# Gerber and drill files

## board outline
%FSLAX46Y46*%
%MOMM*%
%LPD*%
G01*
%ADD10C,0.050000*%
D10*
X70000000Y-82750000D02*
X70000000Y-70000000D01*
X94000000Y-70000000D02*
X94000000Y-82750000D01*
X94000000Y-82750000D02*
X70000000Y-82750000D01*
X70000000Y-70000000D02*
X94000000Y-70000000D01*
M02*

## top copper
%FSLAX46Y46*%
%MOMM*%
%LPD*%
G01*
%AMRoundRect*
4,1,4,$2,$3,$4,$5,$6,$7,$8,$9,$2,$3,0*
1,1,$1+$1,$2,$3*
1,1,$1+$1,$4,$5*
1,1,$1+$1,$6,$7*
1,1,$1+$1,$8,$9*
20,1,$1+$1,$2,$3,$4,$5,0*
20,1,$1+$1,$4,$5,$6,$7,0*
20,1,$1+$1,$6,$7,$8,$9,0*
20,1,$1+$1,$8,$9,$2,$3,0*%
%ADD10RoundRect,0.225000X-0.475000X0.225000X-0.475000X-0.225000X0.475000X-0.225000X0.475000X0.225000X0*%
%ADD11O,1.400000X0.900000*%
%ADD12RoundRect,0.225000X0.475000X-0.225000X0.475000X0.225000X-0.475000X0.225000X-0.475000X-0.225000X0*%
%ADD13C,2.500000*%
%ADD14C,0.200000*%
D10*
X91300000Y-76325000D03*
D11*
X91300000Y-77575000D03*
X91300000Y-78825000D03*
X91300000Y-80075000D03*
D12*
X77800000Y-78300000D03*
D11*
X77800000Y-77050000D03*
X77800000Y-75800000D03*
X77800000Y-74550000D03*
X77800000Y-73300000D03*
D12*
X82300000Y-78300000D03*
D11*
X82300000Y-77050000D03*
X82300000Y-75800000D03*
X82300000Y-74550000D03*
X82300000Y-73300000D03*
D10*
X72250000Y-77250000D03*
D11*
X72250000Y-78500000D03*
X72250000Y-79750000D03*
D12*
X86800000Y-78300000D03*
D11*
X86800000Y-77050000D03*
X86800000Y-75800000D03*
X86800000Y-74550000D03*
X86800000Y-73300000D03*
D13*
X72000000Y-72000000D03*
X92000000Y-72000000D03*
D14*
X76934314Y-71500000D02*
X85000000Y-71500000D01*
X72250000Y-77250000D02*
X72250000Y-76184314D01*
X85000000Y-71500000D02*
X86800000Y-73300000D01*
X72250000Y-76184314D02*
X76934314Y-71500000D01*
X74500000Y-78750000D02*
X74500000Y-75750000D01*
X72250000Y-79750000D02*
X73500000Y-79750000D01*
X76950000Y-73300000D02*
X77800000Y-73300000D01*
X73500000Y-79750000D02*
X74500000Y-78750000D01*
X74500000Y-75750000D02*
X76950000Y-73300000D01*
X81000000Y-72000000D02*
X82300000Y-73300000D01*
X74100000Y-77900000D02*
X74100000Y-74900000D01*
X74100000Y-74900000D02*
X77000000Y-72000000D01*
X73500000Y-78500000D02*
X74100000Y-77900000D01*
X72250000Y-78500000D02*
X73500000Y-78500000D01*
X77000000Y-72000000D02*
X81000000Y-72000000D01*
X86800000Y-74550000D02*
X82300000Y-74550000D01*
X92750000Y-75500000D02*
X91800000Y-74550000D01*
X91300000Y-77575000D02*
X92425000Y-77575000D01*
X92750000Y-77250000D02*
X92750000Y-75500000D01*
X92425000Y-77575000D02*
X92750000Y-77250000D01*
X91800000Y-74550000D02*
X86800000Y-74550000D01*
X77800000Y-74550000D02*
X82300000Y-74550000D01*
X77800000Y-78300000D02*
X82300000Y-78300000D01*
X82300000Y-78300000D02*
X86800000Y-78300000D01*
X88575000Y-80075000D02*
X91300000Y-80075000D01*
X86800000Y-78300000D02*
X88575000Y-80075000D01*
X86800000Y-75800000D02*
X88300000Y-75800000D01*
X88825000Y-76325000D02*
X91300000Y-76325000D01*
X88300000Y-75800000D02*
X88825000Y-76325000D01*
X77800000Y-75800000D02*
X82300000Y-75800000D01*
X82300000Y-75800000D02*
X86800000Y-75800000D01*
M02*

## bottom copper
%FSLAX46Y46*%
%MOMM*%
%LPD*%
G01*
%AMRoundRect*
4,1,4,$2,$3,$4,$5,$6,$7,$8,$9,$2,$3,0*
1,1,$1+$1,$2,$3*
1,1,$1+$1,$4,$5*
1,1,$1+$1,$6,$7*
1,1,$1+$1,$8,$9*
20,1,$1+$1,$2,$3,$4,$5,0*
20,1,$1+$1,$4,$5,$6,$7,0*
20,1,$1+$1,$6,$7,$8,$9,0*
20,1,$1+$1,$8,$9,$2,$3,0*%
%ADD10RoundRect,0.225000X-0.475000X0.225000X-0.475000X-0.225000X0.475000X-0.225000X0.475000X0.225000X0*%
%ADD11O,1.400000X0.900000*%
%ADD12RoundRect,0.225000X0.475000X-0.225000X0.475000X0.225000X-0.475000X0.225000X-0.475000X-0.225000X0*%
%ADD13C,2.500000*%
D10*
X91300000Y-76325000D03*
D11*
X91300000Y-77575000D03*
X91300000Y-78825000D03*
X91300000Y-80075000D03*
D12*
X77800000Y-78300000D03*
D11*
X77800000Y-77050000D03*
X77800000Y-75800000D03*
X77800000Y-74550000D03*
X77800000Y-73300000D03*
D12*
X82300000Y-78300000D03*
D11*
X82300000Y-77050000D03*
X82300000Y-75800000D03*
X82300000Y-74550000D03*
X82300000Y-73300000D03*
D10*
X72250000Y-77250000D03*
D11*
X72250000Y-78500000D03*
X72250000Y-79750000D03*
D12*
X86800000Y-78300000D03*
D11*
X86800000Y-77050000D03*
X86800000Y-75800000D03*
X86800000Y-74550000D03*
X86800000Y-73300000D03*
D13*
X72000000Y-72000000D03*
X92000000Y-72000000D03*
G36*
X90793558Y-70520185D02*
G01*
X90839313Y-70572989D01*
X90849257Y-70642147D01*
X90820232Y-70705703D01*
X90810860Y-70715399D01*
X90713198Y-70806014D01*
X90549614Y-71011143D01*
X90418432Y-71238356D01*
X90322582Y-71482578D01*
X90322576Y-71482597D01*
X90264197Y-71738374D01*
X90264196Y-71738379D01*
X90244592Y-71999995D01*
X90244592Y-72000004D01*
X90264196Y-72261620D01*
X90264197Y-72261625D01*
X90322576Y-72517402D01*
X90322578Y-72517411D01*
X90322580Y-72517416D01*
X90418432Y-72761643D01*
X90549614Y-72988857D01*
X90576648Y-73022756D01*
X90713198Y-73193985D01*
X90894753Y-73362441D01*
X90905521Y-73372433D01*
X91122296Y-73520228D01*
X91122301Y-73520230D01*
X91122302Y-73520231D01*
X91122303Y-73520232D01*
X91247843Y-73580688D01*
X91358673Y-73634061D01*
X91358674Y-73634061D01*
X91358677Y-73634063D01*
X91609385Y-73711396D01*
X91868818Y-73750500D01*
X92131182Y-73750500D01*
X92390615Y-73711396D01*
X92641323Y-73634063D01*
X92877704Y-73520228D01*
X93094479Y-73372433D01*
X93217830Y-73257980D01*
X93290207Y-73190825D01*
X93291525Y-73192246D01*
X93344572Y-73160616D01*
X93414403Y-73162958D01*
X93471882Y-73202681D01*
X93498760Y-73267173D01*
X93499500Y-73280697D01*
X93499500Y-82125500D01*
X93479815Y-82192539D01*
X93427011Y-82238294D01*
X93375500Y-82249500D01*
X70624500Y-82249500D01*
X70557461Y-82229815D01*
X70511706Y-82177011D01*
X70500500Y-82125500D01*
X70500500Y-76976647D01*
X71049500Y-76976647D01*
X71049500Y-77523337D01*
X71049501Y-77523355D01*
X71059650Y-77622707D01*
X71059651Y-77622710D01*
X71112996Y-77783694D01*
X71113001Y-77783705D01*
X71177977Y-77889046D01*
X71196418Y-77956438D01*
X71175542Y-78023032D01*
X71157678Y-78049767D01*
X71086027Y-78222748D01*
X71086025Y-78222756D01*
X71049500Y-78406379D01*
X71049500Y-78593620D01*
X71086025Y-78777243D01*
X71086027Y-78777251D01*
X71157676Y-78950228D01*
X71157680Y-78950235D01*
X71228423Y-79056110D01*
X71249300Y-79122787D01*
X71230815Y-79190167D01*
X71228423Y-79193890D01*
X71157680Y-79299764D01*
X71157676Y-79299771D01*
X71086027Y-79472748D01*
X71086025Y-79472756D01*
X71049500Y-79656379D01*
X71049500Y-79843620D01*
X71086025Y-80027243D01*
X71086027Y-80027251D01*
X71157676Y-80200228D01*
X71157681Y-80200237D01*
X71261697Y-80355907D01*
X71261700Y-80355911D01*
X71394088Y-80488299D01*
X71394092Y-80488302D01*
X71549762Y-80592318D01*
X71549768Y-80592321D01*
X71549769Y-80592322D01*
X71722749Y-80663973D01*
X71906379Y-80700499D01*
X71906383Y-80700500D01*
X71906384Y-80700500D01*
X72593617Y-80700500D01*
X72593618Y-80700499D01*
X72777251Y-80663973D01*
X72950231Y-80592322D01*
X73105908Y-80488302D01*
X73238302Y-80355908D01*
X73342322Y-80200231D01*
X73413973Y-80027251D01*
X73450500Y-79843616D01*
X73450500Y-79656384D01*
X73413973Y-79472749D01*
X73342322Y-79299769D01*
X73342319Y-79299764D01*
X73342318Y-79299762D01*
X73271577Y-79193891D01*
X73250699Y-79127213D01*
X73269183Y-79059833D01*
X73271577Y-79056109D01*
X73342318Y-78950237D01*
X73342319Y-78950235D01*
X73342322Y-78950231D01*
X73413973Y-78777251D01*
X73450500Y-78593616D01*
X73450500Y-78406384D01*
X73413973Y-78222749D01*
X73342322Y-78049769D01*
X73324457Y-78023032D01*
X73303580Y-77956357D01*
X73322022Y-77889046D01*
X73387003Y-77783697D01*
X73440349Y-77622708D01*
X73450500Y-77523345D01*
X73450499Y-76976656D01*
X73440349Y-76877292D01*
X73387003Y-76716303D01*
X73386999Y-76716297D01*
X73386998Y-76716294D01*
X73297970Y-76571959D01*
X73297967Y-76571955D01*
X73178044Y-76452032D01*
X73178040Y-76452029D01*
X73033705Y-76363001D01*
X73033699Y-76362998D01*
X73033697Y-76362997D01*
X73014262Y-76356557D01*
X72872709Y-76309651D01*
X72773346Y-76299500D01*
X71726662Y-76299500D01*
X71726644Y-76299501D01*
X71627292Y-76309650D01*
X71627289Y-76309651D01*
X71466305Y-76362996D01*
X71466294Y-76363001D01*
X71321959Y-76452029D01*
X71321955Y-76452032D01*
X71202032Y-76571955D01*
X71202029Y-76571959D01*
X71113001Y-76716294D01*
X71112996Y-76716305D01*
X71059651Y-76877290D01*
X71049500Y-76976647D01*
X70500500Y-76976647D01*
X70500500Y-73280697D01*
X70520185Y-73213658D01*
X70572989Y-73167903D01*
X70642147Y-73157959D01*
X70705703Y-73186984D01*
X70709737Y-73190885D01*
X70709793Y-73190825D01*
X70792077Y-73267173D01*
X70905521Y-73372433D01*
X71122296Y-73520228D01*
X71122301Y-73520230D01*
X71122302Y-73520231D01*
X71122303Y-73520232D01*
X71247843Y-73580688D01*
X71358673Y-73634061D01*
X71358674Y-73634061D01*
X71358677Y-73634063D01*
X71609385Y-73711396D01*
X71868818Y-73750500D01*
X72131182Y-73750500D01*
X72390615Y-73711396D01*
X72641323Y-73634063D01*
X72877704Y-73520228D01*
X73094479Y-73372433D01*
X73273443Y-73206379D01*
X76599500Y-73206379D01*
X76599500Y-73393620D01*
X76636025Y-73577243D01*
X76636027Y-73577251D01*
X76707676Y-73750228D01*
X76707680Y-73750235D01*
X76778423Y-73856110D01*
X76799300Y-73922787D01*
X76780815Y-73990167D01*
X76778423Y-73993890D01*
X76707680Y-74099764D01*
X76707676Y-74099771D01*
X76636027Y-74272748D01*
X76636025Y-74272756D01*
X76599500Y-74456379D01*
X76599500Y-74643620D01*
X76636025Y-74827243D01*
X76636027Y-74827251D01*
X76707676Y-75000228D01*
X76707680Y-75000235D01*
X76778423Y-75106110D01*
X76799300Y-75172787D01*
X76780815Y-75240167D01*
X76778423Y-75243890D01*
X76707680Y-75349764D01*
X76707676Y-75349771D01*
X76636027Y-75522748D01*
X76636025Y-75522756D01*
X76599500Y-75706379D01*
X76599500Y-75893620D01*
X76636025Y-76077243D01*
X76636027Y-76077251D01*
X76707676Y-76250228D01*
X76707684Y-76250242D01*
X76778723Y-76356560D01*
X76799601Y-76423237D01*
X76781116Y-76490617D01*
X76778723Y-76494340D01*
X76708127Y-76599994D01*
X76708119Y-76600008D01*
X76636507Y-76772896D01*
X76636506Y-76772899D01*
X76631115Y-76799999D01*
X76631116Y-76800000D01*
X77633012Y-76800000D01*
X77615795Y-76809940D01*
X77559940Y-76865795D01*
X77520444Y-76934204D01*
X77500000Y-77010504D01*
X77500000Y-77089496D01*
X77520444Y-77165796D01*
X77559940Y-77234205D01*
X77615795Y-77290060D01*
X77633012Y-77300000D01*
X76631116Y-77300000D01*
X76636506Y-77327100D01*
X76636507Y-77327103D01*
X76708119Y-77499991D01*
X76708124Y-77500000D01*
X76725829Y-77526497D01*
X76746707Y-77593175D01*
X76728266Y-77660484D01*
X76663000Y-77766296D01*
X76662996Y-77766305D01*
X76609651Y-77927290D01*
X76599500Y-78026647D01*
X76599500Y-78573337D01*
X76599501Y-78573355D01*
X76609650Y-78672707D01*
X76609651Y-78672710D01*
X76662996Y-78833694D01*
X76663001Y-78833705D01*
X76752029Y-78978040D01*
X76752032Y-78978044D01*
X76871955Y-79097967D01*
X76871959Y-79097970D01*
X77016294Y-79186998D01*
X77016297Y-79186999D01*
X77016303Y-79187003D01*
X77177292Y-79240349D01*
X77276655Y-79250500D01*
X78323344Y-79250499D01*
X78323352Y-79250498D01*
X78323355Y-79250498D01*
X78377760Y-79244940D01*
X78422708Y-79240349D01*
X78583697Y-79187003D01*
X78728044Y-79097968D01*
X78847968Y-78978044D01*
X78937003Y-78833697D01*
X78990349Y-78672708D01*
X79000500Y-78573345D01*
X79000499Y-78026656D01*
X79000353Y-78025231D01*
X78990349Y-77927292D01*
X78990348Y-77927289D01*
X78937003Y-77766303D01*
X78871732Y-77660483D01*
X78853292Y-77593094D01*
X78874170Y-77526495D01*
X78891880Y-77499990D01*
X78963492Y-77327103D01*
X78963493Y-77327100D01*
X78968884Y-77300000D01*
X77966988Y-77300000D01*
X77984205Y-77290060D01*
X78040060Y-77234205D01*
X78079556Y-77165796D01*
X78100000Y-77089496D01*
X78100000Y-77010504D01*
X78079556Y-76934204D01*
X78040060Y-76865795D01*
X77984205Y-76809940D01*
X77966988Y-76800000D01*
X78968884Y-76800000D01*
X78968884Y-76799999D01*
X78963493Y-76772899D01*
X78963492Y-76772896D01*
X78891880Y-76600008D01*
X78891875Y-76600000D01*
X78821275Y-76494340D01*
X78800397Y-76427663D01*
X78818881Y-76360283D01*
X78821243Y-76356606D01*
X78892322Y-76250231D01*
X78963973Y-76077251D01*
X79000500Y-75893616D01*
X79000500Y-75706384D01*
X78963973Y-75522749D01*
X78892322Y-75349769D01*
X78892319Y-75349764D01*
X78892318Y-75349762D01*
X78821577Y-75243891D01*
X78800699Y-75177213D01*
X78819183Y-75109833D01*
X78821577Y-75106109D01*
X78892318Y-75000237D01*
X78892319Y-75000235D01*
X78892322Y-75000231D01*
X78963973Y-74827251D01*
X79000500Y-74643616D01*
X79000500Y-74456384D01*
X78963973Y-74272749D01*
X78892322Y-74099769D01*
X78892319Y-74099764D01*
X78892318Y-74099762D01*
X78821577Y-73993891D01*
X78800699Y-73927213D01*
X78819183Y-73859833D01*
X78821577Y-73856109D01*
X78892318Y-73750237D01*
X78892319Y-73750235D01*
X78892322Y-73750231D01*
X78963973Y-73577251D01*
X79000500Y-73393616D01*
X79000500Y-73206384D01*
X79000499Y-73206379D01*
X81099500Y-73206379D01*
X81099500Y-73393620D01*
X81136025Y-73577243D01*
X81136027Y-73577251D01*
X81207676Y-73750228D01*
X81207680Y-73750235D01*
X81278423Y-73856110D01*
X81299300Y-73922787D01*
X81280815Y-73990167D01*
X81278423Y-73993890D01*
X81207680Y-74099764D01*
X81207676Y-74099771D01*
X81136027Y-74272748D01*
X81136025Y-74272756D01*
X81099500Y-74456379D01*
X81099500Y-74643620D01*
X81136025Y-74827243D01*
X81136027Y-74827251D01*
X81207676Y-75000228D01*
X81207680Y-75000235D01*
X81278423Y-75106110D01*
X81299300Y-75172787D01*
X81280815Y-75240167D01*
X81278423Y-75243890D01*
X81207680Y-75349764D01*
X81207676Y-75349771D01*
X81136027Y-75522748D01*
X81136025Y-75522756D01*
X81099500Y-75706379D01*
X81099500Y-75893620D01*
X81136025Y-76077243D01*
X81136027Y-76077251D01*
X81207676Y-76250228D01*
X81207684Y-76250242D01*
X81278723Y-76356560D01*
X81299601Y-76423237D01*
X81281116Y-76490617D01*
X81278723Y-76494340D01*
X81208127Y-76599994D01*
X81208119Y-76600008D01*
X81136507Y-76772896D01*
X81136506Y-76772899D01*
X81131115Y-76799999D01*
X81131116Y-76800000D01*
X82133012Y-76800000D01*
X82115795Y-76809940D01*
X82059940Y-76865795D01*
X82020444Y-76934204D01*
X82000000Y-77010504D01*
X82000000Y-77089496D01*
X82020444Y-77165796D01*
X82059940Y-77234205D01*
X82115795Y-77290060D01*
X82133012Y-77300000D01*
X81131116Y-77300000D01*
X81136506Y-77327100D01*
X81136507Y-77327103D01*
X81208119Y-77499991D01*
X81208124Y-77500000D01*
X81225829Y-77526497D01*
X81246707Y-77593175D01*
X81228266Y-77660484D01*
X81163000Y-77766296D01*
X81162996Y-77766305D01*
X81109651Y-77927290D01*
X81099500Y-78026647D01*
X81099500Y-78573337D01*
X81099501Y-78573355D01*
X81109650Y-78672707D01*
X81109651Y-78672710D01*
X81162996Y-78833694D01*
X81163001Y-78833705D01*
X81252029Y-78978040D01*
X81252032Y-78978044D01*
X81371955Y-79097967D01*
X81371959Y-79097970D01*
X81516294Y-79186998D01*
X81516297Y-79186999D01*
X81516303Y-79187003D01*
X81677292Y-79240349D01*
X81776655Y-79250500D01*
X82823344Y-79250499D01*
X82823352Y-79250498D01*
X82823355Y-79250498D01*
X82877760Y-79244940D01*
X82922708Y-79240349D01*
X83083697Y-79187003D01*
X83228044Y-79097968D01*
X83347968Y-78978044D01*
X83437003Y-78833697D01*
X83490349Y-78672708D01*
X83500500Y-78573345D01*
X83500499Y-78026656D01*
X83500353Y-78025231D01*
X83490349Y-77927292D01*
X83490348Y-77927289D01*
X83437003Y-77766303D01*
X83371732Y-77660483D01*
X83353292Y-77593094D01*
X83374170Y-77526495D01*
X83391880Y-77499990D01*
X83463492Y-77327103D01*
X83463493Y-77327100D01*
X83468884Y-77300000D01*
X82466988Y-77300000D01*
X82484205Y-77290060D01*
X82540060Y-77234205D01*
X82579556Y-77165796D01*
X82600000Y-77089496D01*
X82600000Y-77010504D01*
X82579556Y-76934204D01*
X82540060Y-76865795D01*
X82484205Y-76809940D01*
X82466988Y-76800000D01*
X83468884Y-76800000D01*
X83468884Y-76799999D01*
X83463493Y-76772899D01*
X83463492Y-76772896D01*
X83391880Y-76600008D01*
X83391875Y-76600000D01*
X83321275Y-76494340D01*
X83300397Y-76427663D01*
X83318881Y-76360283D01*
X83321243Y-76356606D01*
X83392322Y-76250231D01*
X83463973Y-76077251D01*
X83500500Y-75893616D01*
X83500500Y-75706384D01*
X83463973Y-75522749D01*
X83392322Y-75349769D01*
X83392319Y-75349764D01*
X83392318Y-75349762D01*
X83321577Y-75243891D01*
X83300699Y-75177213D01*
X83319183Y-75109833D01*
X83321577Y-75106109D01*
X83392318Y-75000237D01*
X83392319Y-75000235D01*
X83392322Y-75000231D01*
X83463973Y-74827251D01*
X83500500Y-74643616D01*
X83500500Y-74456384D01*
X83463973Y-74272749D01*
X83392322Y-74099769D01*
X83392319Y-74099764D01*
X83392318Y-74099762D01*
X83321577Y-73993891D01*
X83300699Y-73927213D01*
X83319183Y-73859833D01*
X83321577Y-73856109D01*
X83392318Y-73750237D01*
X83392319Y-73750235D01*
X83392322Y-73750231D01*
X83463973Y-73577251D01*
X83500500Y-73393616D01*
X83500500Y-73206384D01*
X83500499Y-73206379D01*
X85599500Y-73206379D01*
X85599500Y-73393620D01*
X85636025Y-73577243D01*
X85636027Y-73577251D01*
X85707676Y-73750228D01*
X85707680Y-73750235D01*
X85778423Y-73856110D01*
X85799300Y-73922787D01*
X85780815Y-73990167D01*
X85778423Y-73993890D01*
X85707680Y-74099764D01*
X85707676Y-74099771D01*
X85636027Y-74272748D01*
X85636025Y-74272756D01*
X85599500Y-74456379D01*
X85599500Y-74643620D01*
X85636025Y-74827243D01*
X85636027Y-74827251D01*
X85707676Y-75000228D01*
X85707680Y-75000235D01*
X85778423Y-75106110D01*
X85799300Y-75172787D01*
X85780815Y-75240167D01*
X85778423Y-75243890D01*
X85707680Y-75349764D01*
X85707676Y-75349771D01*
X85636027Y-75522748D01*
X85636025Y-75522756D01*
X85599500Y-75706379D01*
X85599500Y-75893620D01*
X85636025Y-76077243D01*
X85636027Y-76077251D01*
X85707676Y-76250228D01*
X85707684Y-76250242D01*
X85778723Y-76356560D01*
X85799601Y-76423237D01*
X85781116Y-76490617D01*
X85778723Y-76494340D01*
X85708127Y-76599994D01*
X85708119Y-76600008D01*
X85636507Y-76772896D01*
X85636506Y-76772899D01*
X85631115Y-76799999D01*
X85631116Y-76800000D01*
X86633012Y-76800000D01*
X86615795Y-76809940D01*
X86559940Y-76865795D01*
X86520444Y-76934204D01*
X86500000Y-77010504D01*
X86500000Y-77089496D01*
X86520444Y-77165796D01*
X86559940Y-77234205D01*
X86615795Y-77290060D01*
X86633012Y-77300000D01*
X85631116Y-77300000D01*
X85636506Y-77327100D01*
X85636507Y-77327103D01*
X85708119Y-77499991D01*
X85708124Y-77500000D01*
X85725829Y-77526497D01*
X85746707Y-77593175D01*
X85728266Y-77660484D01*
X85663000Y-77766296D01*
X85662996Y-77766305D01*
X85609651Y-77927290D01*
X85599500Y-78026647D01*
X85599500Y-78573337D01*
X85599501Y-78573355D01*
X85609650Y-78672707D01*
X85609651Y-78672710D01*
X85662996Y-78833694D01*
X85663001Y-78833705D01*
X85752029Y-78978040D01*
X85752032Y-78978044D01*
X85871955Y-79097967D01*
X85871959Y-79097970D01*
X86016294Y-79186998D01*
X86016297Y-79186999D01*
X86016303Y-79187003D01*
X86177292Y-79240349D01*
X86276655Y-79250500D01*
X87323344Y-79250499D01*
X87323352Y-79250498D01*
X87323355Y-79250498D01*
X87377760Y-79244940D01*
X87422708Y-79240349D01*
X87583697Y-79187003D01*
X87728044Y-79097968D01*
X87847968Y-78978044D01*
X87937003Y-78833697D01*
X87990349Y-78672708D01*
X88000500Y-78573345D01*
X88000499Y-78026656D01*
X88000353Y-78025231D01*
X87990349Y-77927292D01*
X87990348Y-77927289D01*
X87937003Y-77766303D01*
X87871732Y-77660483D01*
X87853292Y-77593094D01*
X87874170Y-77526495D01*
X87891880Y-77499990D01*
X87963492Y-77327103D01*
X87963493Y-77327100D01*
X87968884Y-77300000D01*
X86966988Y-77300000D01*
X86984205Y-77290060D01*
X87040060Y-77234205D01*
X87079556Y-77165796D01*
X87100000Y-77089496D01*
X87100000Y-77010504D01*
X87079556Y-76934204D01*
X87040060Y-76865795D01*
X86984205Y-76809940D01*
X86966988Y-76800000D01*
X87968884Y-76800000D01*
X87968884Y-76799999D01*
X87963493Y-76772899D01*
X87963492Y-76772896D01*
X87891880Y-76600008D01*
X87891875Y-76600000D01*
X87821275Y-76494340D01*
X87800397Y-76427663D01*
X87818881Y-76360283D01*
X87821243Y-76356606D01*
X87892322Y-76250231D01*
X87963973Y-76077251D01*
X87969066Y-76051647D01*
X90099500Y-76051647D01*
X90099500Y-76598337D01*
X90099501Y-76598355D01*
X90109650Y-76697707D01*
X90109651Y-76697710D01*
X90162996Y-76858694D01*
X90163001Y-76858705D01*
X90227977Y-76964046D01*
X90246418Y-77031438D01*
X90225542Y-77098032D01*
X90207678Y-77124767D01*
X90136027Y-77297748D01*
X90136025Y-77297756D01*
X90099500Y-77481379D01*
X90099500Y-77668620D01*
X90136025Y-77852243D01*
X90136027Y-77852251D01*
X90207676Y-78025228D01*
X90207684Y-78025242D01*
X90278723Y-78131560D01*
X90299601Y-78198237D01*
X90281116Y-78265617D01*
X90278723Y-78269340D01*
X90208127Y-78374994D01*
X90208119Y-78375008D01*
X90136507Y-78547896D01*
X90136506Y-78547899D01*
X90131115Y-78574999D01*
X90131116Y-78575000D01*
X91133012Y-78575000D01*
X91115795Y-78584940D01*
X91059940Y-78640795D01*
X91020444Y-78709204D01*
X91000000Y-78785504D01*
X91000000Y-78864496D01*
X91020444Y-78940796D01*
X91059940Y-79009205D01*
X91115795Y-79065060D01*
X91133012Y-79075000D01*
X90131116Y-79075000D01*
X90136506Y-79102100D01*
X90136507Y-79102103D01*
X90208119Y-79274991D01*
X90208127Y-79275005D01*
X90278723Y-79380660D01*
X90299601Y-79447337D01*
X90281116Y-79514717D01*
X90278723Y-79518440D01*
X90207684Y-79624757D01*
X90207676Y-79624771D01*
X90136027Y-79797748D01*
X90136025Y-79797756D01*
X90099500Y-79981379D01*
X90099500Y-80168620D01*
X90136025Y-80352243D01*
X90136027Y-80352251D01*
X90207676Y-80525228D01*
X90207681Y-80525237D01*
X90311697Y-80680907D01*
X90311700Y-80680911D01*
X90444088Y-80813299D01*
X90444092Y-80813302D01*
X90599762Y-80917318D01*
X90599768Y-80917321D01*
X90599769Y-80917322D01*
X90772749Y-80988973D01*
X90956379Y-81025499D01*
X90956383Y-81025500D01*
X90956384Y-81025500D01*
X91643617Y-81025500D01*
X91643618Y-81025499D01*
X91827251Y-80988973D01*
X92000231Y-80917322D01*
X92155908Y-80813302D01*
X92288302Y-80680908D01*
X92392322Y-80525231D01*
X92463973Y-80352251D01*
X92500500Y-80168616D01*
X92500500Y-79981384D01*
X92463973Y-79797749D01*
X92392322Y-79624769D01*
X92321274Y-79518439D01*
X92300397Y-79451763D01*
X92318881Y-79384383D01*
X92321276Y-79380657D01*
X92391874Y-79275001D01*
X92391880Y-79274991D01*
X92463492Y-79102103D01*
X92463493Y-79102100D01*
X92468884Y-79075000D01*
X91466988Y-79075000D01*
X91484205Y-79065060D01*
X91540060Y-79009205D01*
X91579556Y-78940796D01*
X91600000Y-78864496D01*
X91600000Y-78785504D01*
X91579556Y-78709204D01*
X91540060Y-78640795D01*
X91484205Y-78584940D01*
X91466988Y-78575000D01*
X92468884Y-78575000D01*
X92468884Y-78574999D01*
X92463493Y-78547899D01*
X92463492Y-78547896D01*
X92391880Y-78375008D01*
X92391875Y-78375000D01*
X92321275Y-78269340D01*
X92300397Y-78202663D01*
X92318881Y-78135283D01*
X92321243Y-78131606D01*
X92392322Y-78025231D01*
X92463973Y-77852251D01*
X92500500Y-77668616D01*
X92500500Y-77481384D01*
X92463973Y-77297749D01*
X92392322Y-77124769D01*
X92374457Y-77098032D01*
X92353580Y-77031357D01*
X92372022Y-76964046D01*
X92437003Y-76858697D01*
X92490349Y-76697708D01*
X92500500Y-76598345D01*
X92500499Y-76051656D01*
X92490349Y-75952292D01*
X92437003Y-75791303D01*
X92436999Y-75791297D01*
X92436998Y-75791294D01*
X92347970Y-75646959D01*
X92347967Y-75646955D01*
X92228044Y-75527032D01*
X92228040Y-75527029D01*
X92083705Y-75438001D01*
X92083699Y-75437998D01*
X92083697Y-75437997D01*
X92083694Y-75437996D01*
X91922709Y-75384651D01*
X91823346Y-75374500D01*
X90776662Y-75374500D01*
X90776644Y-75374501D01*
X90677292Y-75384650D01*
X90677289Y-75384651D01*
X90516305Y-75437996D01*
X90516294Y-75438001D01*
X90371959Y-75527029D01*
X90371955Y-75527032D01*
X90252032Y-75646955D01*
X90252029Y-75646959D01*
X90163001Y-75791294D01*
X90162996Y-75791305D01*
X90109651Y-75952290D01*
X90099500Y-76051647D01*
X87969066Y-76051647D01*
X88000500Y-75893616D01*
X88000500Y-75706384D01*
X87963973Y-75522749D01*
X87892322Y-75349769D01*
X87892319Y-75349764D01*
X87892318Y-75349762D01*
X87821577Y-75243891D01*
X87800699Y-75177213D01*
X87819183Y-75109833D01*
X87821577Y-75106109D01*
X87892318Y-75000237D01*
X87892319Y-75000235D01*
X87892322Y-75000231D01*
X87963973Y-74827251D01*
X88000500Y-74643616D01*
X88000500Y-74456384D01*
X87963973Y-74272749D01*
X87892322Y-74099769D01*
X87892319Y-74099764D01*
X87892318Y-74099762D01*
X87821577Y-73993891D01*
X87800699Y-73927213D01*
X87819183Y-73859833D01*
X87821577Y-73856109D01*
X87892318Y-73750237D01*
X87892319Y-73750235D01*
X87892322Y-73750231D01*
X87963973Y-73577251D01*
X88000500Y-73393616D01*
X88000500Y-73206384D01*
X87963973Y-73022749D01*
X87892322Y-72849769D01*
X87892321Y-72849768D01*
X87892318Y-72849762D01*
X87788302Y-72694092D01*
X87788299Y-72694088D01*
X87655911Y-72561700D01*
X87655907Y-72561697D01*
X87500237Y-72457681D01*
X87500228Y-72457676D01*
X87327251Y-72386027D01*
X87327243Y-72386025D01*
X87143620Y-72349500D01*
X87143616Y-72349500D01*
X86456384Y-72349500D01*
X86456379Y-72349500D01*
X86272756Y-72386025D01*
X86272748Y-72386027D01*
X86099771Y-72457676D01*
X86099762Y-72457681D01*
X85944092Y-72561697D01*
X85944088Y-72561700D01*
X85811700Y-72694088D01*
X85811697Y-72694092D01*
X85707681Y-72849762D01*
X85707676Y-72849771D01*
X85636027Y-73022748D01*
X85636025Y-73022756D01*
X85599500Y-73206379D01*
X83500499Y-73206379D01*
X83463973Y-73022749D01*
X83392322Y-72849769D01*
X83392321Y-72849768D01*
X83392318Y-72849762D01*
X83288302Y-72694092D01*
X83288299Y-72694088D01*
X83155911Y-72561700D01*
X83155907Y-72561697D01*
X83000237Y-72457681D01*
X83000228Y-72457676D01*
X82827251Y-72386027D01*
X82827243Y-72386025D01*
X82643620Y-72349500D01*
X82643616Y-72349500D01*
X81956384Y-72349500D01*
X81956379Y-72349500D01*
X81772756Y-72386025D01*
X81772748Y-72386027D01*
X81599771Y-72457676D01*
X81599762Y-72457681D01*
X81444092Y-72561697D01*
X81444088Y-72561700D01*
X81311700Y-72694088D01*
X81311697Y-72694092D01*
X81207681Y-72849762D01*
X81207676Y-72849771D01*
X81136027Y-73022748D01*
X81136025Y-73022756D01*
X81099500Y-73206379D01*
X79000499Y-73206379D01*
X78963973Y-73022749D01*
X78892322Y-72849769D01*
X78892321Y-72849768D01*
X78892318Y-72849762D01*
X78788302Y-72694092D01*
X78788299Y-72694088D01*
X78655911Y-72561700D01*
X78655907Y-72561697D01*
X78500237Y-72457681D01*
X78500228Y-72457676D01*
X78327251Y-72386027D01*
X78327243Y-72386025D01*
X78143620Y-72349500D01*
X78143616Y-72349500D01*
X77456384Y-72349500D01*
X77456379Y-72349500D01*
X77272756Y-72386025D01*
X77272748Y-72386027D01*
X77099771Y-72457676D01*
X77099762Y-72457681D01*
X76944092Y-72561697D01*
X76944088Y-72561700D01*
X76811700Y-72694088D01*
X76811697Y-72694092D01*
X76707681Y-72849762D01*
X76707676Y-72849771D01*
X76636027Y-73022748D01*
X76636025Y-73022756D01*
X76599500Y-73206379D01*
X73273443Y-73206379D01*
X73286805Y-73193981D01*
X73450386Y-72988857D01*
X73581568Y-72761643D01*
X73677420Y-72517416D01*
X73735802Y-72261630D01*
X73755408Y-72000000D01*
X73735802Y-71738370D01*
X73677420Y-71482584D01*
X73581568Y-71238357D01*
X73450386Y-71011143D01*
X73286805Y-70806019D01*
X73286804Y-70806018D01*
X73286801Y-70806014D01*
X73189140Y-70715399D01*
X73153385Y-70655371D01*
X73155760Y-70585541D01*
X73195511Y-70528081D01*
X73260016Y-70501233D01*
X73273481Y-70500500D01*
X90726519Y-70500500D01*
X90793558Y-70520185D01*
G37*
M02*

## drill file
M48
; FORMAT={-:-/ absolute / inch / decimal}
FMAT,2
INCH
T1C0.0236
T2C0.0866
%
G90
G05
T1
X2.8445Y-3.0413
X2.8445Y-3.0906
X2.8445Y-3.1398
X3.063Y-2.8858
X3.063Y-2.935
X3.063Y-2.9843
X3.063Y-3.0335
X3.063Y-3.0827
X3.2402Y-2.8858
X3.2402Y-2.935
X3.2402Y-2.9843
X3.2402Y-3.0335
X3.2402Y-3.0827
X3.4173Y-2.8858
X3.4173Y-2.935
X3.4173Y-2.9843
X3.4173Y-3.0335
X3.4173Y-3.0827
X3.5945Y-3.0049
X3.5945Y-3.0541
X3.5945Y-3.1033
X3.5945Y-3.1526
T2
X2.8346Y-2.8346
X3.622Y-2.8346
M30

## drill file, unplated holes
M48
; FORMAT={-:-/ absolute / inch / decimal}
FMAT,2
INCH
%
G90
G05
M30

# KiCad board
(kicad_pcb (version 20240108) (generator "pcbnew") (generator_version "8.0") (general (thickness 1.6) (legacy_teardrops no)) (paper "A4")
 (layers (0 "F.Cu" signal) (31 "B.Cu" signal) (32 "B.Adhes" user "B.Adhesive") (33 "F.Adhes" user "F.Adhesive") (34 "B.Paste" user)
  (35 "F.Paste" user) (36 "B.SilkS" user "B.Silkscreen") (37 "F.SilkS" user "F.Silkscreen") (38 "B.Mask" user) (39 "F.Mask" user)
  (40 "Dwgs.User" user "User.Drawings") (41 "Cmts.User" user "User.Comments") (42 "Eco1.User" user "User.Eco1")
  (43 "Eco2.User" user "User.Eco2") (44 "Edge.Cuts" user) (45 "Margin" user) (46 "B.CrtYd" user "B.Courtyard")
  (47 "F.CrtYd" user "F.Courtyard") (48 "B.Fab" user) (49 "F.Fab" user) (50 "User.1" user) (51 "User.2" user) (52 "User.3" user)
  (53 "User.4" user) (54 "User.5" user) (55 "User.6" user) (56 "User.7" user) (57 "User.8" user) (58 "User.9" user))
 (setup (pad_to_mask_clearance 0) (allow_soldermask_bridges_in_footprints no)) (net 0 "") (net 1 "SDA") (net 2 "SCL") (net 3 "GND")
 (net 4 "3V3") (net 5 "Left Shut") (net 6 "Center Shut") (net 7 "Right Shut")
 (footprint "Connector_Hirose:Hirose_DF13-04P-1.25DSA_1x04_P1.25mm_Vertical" (layer "F.Cu") (at 91.3 76.325 -90)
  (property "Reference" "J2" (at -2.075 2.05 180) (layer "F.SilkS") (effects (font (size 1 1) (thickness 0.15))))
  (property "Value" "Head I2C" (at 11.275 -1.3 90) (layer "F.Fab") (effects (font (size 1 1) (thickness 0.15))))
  (pad "1" thru_hole roundrect (at 0 0 270) (size 0.9 1.4) (drill 0.6) (layers "*.Cu" "*.Mask") (remove_unused_layers no)
   (roundrect_rratio 0.25) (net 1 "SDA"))
  (pad "2" thru_hole oval (at 1.25 0 270) (size 0.9 1.4) (drill 0.6) (layers "*.Cu" "*.Mask") (remove_unused_layers no) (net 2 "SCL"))
  (pad "3" thru_hole oval (at 2.5 0 270) (size 0.9 1.4) (drill 0.6) (layers "*.Cu" "*.Mask") (remove_unused_layers no) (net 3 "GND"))
  (pad "4" thru_hole oval (at 3.75 0 270) (size 0.9 1.4) (drill 0.6) (layers "*.Cu" "*.Mask") (remove_unused_layers no) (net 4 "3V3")))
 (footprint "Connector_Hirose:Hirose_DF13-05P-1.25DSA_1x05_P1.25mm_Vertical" (layer "F.Cu") (at 77.8 78.3 90)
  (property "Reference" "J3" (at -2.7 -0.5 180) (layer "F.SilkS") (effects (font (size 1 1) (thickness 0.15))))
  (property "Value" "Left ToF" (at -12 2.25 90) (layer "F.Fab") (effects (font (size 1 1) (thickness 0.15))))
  (pad "1" thru_hole roundrect (at 0 0 90) (size 0.9 1.4) (drill 0.6) (layers "*.Cu" "*.Mask") (remove_unused_layers no)
   (roundrect_rratio 0.25) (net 4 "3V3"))
  (pad "2" thru_hole oval (at 1.25 0 90) (size 0.9 1.4) (drill 0.6) (layers "*.Cu" "*.Mask") (remove_unused_layers no) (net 3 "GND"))
  (pad "3" thru_hole oval (at 2.5 0 90) (size 0.9 1.4) (drill 0.6) (layers "*.Cu" "*.Mask") (remove_unused_layers no) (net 1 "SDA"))
  (pad "4" thru_hole oval (at 3.75 0 90) (size 0.9 1.4) (drill 0.6) (layers "*.Cu" "*.Mask") (remove_unused_layers no) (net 2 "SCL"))
  (pad "5" thru_hole oval (at 5 0 90) (size 0.9 1.4) (drill 0.6) (layers "*.Cu" "*.Mask") (remove_unused_layers no) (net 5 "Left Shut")))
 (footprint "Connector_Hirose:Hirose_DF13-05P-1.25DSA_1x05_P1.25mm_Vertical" (layer "F.Cu") (at 82.3 78.3 90)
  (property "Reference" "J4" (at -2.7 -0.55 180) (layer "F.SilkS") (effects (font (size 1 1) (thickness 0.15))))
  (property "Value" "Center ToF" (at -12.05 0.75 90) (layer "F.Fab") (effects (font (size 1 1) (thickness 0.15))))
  (pad "1" thru_hole roundrect (at 0 0 90) (size 0.9 1.4) (drill 0.6) (layers "*.Cu" "*.Mask") (remove_unused_layers no)
   (roundrect_rratio 0.25) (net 4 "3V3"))
  (pad "2" thru_hole oval (at 1.25 0 90) (size 0.9 1.4) (drill 0.6) (layers "*.Cu" "*.Mask") (remove_unused_layers no) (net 3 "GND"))
  (pad "3" thru_hole oval (at 2.5 0 90) (size 0.9 1.4) (drill 0.6) (layers "*.Cu" "*.Mask") (remove_unused_layers no) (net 1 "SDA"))
  (pad "4" thru_hole oval (at 3.75 0 90) (size 0.9 1.4) (drill 0.6) (layers "*.Cu" "*.Mask") (remove_unused_layers no) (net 2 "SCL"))
  (pad "5" thru_hole oval (at 5 0 90) (size 0.9 1.4) (drill 0.6) (layers "*.Cu" "*.Mask") (remove_unused_layers no) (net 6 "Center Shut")))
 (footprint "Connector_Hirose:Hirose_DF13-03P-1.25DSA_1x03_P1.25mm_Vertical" (layer "F.Cu") (at 72.25 77.25 -90)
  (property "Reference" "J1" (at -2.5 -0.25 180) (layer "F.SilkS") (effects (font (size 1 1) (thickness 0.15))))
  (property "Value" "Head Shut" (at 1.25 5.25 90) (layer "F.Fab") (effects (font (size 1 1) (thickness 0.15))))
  (pad "1" thru_hole roundrect (at 0 0 270) (size 0.9 1.4) (drill 0.6) (layers "*.Cu" "*.Mask") (remove_unused_layers no)
   (roundrect_rratio 0.25) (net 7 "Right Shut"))
  (pad "2" thru_hole oval (at 1.25 0 270) (size 0.9 1.4) (drill 0.6) (layers "*.Cu" "*.Mask") (remove_unused_layers no)
   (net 6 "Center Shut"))
  (pad "3" thru_hole oval (at 2.5 0 270) (size 0.9 1.4) (drill 0.6) (layers "*.Cu" "*.Mask") (remove_unused_layers no) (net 5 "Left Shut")))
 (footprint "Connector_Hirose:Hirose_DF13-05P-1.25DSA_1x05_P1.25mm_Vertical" (layer "F.Cu") (at 86.8 78.3 90)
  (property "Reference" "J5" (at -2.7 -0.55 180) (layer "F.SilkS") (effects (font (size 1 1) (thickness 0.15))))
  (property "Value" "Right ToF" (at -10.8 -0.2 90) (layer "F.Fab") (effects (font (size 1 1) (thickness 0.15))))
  (pad "1" thru_hole roundrect (at 0 0 90) (size 0.9 1.4) (drill 0.6) (layers "*.Cu" "*.Mask") (remove_unused_layers no)
   (roundrect_rratio 0.25) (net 4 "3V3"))
  (pad "2" thru_hole oval (at 1.25 0 90) (size 0.9 1.4) (drill 0.6) (layers "*.Cu" "*.Mask") (remove_unused_layers no) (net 3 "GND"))
  (pad "3" thru_hole oval (at 2.5 0 90) (size 0.9 1.4) (drill 0.6) (layers "*.Cu" "*.Mask") (remove_unused_layers no) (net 1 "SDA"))
  (pad "4" thru_hole oval (at 3.75 0 90) (size 0.9 1.4) (drill 0.6) (layers "*.Cu" "*.Mask") (remove_unused_layers no) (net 2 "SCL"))
  (pad "5" thru_hole oval (at 5 0 90) (size 0.9 1.4) (drill 0.6) (layers "*.Cu" "*.Mask") (remove_unused_layers no) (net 7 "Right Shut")))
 (gr_line (start 70 82.75) (end 70 70) (stroke (width 0.05) (type default)) (layer "Edge.Cuts"))
 (gr_line (start 94 70) (end 94 82.75) (stroke (width 0.05) (type default)) (layer "Edge.Cuts"))
 (gr_line (start 94 82.75) (end 70 82.75) (stroke (width 0.05) (type default)) (layer "Edge.Cuts"))
 (gr_line (start 70 70) (end 94 70) (stroke (width 0.05) (type default)) (layer "Edge.Cuts"))
 (via (at 72 72) (size 2.5) (drill 2.2) (layers "F.Cu" "B.Cu") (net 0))
 (via (at 92 72) (size 2.5) (drill 2.2) (layers "F.Cu" "B.Cu") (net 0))
 (segment (start 76.934314 71.5) (end 85 71.5) (width 0.2) (layer "F.Cu") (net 7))
 (segment (start 72.25 77.25) (end 72.25 76.184314) (width 0.2) (layer "F.Cu") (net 7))
 (segment (start 85 71.5) (end 86.8 73.3) (width 0.2) (layer "F.Cu") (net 7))
 (segment (start 72.25 76.184314) (end 76.934314 71.5) (width 0.2) (layer "F.Cu") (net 7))
 (segment (start 74.5 78.75) (end 74.5 75.75) (width 0.2) (layer "F.Cu") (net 5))
 (segment (start 72.25 79.75) (end 73.5 79.75) (width 0.2) (layer "F.Cu") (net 5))
 (segment (start 76.95 73.3) (end 77.8 73.3) (width 0.2) (layer "F.Cu") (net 5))
 (segment (start 73.5 79.75) (end 74.5 78.75) (width 0.2) (layer "F.Cu") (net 5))
 (segment (start 74.5 75.75) (end 76.95 73.3) (width 0.2) (layer "F.Cu") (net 5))
 (segment (start 81 72) (end 82.3 73.3) (width 0.2) (layer "F.Cu") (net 6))
 (segment (start 74.1 77.9) (end 74.1 74.9) (width 0.2) (layer "F.Cu") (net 6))
 (segment (start 74.1 74.9) (end 77 72) (width 0.2) (layer "F.Cu") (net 6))
 (segment (start 73.5 78.5) (end 74.1 77.9) (width 0.2) (layer "F.Cu") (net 6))
 (segment (start 72.25 78.5) (end 73.5 78.5) (width 0.2) (layer "F.Cu") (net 6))
 (segment (start 77 72) (end 81 72) (width 0.2) (layer "F.Cu") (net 6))
 (segment (start 86.8 74.55) (end 82.3 74.55) (width 0.2) (layer "F.Cu") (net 2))
 (segment (start 92.75 75.5) (end 91.8 74.55) (width 0.2) (layer "F.Cu") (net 2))
 (segment (start 91.3 77.575) (end 92.425 77.575) (width 0.2) (layer "F.Cu") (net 2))
 (segment (start 92.75 77.25) (end 92.75 75.5) (width 0.2) (layer "F.Cu") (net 2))
 (segment (start 92.425 77.575) (end 92.75 77.25) (width 0.2) (layer "F.Cu") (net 2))
 (segment (start 91.8 74.55) (end 86.8 74.55) (width 0.2) (layer "F.Cu") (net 2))
 (segment (start 77.8 74.55) (end 82.3 74.55) (width 0.2) (layer "F.Cu") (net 2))
 (segment (start 77.8 78.3) (end 82.3 78.3) (width 0.2) (layer "F.Cu") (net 4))
 (segment (start 82.3 78.3) (end 86.8 78.3) (width 0.2) (layer "F.Cu") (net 4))
 (segment (start 88.575 80.075) (end 91.3 80.075) (width 0.2) (layer "F.Cu") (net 4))
 (segment (start 86.8 78.3) (end 88.575 80.075) (width 0.2) (layer "F.Cu") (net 4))
 (segment (start 86.8 75.8) (end 88.3 75.8) (width 0.2) (layer "F.Cu") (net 1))
 (segment (start 88.825 76.325) (end 91.3 76.325) (width 0.2) (layer "F.Cu") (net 1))
 (segment (start 88.3 75.8) (end 88.825 76.325) (width 0.2) (layer "F.Cu") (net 1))
 (segment (start 77.8 75.8) (end 82.3 75.8) (width 0.2) (layer "F.Cu") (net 1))
 (segment (start 82.3 75.8) (end 86.8 75.8) (width 0.2) (layer "F.Cu") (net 1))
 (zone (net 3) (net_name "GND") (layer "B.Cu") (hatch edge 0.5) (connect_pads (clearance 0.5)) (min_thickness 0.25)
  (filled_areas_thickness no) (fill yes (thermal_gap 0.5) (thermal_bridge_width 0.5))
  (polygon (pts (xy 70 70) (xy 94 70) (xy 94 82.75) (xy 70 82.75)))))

